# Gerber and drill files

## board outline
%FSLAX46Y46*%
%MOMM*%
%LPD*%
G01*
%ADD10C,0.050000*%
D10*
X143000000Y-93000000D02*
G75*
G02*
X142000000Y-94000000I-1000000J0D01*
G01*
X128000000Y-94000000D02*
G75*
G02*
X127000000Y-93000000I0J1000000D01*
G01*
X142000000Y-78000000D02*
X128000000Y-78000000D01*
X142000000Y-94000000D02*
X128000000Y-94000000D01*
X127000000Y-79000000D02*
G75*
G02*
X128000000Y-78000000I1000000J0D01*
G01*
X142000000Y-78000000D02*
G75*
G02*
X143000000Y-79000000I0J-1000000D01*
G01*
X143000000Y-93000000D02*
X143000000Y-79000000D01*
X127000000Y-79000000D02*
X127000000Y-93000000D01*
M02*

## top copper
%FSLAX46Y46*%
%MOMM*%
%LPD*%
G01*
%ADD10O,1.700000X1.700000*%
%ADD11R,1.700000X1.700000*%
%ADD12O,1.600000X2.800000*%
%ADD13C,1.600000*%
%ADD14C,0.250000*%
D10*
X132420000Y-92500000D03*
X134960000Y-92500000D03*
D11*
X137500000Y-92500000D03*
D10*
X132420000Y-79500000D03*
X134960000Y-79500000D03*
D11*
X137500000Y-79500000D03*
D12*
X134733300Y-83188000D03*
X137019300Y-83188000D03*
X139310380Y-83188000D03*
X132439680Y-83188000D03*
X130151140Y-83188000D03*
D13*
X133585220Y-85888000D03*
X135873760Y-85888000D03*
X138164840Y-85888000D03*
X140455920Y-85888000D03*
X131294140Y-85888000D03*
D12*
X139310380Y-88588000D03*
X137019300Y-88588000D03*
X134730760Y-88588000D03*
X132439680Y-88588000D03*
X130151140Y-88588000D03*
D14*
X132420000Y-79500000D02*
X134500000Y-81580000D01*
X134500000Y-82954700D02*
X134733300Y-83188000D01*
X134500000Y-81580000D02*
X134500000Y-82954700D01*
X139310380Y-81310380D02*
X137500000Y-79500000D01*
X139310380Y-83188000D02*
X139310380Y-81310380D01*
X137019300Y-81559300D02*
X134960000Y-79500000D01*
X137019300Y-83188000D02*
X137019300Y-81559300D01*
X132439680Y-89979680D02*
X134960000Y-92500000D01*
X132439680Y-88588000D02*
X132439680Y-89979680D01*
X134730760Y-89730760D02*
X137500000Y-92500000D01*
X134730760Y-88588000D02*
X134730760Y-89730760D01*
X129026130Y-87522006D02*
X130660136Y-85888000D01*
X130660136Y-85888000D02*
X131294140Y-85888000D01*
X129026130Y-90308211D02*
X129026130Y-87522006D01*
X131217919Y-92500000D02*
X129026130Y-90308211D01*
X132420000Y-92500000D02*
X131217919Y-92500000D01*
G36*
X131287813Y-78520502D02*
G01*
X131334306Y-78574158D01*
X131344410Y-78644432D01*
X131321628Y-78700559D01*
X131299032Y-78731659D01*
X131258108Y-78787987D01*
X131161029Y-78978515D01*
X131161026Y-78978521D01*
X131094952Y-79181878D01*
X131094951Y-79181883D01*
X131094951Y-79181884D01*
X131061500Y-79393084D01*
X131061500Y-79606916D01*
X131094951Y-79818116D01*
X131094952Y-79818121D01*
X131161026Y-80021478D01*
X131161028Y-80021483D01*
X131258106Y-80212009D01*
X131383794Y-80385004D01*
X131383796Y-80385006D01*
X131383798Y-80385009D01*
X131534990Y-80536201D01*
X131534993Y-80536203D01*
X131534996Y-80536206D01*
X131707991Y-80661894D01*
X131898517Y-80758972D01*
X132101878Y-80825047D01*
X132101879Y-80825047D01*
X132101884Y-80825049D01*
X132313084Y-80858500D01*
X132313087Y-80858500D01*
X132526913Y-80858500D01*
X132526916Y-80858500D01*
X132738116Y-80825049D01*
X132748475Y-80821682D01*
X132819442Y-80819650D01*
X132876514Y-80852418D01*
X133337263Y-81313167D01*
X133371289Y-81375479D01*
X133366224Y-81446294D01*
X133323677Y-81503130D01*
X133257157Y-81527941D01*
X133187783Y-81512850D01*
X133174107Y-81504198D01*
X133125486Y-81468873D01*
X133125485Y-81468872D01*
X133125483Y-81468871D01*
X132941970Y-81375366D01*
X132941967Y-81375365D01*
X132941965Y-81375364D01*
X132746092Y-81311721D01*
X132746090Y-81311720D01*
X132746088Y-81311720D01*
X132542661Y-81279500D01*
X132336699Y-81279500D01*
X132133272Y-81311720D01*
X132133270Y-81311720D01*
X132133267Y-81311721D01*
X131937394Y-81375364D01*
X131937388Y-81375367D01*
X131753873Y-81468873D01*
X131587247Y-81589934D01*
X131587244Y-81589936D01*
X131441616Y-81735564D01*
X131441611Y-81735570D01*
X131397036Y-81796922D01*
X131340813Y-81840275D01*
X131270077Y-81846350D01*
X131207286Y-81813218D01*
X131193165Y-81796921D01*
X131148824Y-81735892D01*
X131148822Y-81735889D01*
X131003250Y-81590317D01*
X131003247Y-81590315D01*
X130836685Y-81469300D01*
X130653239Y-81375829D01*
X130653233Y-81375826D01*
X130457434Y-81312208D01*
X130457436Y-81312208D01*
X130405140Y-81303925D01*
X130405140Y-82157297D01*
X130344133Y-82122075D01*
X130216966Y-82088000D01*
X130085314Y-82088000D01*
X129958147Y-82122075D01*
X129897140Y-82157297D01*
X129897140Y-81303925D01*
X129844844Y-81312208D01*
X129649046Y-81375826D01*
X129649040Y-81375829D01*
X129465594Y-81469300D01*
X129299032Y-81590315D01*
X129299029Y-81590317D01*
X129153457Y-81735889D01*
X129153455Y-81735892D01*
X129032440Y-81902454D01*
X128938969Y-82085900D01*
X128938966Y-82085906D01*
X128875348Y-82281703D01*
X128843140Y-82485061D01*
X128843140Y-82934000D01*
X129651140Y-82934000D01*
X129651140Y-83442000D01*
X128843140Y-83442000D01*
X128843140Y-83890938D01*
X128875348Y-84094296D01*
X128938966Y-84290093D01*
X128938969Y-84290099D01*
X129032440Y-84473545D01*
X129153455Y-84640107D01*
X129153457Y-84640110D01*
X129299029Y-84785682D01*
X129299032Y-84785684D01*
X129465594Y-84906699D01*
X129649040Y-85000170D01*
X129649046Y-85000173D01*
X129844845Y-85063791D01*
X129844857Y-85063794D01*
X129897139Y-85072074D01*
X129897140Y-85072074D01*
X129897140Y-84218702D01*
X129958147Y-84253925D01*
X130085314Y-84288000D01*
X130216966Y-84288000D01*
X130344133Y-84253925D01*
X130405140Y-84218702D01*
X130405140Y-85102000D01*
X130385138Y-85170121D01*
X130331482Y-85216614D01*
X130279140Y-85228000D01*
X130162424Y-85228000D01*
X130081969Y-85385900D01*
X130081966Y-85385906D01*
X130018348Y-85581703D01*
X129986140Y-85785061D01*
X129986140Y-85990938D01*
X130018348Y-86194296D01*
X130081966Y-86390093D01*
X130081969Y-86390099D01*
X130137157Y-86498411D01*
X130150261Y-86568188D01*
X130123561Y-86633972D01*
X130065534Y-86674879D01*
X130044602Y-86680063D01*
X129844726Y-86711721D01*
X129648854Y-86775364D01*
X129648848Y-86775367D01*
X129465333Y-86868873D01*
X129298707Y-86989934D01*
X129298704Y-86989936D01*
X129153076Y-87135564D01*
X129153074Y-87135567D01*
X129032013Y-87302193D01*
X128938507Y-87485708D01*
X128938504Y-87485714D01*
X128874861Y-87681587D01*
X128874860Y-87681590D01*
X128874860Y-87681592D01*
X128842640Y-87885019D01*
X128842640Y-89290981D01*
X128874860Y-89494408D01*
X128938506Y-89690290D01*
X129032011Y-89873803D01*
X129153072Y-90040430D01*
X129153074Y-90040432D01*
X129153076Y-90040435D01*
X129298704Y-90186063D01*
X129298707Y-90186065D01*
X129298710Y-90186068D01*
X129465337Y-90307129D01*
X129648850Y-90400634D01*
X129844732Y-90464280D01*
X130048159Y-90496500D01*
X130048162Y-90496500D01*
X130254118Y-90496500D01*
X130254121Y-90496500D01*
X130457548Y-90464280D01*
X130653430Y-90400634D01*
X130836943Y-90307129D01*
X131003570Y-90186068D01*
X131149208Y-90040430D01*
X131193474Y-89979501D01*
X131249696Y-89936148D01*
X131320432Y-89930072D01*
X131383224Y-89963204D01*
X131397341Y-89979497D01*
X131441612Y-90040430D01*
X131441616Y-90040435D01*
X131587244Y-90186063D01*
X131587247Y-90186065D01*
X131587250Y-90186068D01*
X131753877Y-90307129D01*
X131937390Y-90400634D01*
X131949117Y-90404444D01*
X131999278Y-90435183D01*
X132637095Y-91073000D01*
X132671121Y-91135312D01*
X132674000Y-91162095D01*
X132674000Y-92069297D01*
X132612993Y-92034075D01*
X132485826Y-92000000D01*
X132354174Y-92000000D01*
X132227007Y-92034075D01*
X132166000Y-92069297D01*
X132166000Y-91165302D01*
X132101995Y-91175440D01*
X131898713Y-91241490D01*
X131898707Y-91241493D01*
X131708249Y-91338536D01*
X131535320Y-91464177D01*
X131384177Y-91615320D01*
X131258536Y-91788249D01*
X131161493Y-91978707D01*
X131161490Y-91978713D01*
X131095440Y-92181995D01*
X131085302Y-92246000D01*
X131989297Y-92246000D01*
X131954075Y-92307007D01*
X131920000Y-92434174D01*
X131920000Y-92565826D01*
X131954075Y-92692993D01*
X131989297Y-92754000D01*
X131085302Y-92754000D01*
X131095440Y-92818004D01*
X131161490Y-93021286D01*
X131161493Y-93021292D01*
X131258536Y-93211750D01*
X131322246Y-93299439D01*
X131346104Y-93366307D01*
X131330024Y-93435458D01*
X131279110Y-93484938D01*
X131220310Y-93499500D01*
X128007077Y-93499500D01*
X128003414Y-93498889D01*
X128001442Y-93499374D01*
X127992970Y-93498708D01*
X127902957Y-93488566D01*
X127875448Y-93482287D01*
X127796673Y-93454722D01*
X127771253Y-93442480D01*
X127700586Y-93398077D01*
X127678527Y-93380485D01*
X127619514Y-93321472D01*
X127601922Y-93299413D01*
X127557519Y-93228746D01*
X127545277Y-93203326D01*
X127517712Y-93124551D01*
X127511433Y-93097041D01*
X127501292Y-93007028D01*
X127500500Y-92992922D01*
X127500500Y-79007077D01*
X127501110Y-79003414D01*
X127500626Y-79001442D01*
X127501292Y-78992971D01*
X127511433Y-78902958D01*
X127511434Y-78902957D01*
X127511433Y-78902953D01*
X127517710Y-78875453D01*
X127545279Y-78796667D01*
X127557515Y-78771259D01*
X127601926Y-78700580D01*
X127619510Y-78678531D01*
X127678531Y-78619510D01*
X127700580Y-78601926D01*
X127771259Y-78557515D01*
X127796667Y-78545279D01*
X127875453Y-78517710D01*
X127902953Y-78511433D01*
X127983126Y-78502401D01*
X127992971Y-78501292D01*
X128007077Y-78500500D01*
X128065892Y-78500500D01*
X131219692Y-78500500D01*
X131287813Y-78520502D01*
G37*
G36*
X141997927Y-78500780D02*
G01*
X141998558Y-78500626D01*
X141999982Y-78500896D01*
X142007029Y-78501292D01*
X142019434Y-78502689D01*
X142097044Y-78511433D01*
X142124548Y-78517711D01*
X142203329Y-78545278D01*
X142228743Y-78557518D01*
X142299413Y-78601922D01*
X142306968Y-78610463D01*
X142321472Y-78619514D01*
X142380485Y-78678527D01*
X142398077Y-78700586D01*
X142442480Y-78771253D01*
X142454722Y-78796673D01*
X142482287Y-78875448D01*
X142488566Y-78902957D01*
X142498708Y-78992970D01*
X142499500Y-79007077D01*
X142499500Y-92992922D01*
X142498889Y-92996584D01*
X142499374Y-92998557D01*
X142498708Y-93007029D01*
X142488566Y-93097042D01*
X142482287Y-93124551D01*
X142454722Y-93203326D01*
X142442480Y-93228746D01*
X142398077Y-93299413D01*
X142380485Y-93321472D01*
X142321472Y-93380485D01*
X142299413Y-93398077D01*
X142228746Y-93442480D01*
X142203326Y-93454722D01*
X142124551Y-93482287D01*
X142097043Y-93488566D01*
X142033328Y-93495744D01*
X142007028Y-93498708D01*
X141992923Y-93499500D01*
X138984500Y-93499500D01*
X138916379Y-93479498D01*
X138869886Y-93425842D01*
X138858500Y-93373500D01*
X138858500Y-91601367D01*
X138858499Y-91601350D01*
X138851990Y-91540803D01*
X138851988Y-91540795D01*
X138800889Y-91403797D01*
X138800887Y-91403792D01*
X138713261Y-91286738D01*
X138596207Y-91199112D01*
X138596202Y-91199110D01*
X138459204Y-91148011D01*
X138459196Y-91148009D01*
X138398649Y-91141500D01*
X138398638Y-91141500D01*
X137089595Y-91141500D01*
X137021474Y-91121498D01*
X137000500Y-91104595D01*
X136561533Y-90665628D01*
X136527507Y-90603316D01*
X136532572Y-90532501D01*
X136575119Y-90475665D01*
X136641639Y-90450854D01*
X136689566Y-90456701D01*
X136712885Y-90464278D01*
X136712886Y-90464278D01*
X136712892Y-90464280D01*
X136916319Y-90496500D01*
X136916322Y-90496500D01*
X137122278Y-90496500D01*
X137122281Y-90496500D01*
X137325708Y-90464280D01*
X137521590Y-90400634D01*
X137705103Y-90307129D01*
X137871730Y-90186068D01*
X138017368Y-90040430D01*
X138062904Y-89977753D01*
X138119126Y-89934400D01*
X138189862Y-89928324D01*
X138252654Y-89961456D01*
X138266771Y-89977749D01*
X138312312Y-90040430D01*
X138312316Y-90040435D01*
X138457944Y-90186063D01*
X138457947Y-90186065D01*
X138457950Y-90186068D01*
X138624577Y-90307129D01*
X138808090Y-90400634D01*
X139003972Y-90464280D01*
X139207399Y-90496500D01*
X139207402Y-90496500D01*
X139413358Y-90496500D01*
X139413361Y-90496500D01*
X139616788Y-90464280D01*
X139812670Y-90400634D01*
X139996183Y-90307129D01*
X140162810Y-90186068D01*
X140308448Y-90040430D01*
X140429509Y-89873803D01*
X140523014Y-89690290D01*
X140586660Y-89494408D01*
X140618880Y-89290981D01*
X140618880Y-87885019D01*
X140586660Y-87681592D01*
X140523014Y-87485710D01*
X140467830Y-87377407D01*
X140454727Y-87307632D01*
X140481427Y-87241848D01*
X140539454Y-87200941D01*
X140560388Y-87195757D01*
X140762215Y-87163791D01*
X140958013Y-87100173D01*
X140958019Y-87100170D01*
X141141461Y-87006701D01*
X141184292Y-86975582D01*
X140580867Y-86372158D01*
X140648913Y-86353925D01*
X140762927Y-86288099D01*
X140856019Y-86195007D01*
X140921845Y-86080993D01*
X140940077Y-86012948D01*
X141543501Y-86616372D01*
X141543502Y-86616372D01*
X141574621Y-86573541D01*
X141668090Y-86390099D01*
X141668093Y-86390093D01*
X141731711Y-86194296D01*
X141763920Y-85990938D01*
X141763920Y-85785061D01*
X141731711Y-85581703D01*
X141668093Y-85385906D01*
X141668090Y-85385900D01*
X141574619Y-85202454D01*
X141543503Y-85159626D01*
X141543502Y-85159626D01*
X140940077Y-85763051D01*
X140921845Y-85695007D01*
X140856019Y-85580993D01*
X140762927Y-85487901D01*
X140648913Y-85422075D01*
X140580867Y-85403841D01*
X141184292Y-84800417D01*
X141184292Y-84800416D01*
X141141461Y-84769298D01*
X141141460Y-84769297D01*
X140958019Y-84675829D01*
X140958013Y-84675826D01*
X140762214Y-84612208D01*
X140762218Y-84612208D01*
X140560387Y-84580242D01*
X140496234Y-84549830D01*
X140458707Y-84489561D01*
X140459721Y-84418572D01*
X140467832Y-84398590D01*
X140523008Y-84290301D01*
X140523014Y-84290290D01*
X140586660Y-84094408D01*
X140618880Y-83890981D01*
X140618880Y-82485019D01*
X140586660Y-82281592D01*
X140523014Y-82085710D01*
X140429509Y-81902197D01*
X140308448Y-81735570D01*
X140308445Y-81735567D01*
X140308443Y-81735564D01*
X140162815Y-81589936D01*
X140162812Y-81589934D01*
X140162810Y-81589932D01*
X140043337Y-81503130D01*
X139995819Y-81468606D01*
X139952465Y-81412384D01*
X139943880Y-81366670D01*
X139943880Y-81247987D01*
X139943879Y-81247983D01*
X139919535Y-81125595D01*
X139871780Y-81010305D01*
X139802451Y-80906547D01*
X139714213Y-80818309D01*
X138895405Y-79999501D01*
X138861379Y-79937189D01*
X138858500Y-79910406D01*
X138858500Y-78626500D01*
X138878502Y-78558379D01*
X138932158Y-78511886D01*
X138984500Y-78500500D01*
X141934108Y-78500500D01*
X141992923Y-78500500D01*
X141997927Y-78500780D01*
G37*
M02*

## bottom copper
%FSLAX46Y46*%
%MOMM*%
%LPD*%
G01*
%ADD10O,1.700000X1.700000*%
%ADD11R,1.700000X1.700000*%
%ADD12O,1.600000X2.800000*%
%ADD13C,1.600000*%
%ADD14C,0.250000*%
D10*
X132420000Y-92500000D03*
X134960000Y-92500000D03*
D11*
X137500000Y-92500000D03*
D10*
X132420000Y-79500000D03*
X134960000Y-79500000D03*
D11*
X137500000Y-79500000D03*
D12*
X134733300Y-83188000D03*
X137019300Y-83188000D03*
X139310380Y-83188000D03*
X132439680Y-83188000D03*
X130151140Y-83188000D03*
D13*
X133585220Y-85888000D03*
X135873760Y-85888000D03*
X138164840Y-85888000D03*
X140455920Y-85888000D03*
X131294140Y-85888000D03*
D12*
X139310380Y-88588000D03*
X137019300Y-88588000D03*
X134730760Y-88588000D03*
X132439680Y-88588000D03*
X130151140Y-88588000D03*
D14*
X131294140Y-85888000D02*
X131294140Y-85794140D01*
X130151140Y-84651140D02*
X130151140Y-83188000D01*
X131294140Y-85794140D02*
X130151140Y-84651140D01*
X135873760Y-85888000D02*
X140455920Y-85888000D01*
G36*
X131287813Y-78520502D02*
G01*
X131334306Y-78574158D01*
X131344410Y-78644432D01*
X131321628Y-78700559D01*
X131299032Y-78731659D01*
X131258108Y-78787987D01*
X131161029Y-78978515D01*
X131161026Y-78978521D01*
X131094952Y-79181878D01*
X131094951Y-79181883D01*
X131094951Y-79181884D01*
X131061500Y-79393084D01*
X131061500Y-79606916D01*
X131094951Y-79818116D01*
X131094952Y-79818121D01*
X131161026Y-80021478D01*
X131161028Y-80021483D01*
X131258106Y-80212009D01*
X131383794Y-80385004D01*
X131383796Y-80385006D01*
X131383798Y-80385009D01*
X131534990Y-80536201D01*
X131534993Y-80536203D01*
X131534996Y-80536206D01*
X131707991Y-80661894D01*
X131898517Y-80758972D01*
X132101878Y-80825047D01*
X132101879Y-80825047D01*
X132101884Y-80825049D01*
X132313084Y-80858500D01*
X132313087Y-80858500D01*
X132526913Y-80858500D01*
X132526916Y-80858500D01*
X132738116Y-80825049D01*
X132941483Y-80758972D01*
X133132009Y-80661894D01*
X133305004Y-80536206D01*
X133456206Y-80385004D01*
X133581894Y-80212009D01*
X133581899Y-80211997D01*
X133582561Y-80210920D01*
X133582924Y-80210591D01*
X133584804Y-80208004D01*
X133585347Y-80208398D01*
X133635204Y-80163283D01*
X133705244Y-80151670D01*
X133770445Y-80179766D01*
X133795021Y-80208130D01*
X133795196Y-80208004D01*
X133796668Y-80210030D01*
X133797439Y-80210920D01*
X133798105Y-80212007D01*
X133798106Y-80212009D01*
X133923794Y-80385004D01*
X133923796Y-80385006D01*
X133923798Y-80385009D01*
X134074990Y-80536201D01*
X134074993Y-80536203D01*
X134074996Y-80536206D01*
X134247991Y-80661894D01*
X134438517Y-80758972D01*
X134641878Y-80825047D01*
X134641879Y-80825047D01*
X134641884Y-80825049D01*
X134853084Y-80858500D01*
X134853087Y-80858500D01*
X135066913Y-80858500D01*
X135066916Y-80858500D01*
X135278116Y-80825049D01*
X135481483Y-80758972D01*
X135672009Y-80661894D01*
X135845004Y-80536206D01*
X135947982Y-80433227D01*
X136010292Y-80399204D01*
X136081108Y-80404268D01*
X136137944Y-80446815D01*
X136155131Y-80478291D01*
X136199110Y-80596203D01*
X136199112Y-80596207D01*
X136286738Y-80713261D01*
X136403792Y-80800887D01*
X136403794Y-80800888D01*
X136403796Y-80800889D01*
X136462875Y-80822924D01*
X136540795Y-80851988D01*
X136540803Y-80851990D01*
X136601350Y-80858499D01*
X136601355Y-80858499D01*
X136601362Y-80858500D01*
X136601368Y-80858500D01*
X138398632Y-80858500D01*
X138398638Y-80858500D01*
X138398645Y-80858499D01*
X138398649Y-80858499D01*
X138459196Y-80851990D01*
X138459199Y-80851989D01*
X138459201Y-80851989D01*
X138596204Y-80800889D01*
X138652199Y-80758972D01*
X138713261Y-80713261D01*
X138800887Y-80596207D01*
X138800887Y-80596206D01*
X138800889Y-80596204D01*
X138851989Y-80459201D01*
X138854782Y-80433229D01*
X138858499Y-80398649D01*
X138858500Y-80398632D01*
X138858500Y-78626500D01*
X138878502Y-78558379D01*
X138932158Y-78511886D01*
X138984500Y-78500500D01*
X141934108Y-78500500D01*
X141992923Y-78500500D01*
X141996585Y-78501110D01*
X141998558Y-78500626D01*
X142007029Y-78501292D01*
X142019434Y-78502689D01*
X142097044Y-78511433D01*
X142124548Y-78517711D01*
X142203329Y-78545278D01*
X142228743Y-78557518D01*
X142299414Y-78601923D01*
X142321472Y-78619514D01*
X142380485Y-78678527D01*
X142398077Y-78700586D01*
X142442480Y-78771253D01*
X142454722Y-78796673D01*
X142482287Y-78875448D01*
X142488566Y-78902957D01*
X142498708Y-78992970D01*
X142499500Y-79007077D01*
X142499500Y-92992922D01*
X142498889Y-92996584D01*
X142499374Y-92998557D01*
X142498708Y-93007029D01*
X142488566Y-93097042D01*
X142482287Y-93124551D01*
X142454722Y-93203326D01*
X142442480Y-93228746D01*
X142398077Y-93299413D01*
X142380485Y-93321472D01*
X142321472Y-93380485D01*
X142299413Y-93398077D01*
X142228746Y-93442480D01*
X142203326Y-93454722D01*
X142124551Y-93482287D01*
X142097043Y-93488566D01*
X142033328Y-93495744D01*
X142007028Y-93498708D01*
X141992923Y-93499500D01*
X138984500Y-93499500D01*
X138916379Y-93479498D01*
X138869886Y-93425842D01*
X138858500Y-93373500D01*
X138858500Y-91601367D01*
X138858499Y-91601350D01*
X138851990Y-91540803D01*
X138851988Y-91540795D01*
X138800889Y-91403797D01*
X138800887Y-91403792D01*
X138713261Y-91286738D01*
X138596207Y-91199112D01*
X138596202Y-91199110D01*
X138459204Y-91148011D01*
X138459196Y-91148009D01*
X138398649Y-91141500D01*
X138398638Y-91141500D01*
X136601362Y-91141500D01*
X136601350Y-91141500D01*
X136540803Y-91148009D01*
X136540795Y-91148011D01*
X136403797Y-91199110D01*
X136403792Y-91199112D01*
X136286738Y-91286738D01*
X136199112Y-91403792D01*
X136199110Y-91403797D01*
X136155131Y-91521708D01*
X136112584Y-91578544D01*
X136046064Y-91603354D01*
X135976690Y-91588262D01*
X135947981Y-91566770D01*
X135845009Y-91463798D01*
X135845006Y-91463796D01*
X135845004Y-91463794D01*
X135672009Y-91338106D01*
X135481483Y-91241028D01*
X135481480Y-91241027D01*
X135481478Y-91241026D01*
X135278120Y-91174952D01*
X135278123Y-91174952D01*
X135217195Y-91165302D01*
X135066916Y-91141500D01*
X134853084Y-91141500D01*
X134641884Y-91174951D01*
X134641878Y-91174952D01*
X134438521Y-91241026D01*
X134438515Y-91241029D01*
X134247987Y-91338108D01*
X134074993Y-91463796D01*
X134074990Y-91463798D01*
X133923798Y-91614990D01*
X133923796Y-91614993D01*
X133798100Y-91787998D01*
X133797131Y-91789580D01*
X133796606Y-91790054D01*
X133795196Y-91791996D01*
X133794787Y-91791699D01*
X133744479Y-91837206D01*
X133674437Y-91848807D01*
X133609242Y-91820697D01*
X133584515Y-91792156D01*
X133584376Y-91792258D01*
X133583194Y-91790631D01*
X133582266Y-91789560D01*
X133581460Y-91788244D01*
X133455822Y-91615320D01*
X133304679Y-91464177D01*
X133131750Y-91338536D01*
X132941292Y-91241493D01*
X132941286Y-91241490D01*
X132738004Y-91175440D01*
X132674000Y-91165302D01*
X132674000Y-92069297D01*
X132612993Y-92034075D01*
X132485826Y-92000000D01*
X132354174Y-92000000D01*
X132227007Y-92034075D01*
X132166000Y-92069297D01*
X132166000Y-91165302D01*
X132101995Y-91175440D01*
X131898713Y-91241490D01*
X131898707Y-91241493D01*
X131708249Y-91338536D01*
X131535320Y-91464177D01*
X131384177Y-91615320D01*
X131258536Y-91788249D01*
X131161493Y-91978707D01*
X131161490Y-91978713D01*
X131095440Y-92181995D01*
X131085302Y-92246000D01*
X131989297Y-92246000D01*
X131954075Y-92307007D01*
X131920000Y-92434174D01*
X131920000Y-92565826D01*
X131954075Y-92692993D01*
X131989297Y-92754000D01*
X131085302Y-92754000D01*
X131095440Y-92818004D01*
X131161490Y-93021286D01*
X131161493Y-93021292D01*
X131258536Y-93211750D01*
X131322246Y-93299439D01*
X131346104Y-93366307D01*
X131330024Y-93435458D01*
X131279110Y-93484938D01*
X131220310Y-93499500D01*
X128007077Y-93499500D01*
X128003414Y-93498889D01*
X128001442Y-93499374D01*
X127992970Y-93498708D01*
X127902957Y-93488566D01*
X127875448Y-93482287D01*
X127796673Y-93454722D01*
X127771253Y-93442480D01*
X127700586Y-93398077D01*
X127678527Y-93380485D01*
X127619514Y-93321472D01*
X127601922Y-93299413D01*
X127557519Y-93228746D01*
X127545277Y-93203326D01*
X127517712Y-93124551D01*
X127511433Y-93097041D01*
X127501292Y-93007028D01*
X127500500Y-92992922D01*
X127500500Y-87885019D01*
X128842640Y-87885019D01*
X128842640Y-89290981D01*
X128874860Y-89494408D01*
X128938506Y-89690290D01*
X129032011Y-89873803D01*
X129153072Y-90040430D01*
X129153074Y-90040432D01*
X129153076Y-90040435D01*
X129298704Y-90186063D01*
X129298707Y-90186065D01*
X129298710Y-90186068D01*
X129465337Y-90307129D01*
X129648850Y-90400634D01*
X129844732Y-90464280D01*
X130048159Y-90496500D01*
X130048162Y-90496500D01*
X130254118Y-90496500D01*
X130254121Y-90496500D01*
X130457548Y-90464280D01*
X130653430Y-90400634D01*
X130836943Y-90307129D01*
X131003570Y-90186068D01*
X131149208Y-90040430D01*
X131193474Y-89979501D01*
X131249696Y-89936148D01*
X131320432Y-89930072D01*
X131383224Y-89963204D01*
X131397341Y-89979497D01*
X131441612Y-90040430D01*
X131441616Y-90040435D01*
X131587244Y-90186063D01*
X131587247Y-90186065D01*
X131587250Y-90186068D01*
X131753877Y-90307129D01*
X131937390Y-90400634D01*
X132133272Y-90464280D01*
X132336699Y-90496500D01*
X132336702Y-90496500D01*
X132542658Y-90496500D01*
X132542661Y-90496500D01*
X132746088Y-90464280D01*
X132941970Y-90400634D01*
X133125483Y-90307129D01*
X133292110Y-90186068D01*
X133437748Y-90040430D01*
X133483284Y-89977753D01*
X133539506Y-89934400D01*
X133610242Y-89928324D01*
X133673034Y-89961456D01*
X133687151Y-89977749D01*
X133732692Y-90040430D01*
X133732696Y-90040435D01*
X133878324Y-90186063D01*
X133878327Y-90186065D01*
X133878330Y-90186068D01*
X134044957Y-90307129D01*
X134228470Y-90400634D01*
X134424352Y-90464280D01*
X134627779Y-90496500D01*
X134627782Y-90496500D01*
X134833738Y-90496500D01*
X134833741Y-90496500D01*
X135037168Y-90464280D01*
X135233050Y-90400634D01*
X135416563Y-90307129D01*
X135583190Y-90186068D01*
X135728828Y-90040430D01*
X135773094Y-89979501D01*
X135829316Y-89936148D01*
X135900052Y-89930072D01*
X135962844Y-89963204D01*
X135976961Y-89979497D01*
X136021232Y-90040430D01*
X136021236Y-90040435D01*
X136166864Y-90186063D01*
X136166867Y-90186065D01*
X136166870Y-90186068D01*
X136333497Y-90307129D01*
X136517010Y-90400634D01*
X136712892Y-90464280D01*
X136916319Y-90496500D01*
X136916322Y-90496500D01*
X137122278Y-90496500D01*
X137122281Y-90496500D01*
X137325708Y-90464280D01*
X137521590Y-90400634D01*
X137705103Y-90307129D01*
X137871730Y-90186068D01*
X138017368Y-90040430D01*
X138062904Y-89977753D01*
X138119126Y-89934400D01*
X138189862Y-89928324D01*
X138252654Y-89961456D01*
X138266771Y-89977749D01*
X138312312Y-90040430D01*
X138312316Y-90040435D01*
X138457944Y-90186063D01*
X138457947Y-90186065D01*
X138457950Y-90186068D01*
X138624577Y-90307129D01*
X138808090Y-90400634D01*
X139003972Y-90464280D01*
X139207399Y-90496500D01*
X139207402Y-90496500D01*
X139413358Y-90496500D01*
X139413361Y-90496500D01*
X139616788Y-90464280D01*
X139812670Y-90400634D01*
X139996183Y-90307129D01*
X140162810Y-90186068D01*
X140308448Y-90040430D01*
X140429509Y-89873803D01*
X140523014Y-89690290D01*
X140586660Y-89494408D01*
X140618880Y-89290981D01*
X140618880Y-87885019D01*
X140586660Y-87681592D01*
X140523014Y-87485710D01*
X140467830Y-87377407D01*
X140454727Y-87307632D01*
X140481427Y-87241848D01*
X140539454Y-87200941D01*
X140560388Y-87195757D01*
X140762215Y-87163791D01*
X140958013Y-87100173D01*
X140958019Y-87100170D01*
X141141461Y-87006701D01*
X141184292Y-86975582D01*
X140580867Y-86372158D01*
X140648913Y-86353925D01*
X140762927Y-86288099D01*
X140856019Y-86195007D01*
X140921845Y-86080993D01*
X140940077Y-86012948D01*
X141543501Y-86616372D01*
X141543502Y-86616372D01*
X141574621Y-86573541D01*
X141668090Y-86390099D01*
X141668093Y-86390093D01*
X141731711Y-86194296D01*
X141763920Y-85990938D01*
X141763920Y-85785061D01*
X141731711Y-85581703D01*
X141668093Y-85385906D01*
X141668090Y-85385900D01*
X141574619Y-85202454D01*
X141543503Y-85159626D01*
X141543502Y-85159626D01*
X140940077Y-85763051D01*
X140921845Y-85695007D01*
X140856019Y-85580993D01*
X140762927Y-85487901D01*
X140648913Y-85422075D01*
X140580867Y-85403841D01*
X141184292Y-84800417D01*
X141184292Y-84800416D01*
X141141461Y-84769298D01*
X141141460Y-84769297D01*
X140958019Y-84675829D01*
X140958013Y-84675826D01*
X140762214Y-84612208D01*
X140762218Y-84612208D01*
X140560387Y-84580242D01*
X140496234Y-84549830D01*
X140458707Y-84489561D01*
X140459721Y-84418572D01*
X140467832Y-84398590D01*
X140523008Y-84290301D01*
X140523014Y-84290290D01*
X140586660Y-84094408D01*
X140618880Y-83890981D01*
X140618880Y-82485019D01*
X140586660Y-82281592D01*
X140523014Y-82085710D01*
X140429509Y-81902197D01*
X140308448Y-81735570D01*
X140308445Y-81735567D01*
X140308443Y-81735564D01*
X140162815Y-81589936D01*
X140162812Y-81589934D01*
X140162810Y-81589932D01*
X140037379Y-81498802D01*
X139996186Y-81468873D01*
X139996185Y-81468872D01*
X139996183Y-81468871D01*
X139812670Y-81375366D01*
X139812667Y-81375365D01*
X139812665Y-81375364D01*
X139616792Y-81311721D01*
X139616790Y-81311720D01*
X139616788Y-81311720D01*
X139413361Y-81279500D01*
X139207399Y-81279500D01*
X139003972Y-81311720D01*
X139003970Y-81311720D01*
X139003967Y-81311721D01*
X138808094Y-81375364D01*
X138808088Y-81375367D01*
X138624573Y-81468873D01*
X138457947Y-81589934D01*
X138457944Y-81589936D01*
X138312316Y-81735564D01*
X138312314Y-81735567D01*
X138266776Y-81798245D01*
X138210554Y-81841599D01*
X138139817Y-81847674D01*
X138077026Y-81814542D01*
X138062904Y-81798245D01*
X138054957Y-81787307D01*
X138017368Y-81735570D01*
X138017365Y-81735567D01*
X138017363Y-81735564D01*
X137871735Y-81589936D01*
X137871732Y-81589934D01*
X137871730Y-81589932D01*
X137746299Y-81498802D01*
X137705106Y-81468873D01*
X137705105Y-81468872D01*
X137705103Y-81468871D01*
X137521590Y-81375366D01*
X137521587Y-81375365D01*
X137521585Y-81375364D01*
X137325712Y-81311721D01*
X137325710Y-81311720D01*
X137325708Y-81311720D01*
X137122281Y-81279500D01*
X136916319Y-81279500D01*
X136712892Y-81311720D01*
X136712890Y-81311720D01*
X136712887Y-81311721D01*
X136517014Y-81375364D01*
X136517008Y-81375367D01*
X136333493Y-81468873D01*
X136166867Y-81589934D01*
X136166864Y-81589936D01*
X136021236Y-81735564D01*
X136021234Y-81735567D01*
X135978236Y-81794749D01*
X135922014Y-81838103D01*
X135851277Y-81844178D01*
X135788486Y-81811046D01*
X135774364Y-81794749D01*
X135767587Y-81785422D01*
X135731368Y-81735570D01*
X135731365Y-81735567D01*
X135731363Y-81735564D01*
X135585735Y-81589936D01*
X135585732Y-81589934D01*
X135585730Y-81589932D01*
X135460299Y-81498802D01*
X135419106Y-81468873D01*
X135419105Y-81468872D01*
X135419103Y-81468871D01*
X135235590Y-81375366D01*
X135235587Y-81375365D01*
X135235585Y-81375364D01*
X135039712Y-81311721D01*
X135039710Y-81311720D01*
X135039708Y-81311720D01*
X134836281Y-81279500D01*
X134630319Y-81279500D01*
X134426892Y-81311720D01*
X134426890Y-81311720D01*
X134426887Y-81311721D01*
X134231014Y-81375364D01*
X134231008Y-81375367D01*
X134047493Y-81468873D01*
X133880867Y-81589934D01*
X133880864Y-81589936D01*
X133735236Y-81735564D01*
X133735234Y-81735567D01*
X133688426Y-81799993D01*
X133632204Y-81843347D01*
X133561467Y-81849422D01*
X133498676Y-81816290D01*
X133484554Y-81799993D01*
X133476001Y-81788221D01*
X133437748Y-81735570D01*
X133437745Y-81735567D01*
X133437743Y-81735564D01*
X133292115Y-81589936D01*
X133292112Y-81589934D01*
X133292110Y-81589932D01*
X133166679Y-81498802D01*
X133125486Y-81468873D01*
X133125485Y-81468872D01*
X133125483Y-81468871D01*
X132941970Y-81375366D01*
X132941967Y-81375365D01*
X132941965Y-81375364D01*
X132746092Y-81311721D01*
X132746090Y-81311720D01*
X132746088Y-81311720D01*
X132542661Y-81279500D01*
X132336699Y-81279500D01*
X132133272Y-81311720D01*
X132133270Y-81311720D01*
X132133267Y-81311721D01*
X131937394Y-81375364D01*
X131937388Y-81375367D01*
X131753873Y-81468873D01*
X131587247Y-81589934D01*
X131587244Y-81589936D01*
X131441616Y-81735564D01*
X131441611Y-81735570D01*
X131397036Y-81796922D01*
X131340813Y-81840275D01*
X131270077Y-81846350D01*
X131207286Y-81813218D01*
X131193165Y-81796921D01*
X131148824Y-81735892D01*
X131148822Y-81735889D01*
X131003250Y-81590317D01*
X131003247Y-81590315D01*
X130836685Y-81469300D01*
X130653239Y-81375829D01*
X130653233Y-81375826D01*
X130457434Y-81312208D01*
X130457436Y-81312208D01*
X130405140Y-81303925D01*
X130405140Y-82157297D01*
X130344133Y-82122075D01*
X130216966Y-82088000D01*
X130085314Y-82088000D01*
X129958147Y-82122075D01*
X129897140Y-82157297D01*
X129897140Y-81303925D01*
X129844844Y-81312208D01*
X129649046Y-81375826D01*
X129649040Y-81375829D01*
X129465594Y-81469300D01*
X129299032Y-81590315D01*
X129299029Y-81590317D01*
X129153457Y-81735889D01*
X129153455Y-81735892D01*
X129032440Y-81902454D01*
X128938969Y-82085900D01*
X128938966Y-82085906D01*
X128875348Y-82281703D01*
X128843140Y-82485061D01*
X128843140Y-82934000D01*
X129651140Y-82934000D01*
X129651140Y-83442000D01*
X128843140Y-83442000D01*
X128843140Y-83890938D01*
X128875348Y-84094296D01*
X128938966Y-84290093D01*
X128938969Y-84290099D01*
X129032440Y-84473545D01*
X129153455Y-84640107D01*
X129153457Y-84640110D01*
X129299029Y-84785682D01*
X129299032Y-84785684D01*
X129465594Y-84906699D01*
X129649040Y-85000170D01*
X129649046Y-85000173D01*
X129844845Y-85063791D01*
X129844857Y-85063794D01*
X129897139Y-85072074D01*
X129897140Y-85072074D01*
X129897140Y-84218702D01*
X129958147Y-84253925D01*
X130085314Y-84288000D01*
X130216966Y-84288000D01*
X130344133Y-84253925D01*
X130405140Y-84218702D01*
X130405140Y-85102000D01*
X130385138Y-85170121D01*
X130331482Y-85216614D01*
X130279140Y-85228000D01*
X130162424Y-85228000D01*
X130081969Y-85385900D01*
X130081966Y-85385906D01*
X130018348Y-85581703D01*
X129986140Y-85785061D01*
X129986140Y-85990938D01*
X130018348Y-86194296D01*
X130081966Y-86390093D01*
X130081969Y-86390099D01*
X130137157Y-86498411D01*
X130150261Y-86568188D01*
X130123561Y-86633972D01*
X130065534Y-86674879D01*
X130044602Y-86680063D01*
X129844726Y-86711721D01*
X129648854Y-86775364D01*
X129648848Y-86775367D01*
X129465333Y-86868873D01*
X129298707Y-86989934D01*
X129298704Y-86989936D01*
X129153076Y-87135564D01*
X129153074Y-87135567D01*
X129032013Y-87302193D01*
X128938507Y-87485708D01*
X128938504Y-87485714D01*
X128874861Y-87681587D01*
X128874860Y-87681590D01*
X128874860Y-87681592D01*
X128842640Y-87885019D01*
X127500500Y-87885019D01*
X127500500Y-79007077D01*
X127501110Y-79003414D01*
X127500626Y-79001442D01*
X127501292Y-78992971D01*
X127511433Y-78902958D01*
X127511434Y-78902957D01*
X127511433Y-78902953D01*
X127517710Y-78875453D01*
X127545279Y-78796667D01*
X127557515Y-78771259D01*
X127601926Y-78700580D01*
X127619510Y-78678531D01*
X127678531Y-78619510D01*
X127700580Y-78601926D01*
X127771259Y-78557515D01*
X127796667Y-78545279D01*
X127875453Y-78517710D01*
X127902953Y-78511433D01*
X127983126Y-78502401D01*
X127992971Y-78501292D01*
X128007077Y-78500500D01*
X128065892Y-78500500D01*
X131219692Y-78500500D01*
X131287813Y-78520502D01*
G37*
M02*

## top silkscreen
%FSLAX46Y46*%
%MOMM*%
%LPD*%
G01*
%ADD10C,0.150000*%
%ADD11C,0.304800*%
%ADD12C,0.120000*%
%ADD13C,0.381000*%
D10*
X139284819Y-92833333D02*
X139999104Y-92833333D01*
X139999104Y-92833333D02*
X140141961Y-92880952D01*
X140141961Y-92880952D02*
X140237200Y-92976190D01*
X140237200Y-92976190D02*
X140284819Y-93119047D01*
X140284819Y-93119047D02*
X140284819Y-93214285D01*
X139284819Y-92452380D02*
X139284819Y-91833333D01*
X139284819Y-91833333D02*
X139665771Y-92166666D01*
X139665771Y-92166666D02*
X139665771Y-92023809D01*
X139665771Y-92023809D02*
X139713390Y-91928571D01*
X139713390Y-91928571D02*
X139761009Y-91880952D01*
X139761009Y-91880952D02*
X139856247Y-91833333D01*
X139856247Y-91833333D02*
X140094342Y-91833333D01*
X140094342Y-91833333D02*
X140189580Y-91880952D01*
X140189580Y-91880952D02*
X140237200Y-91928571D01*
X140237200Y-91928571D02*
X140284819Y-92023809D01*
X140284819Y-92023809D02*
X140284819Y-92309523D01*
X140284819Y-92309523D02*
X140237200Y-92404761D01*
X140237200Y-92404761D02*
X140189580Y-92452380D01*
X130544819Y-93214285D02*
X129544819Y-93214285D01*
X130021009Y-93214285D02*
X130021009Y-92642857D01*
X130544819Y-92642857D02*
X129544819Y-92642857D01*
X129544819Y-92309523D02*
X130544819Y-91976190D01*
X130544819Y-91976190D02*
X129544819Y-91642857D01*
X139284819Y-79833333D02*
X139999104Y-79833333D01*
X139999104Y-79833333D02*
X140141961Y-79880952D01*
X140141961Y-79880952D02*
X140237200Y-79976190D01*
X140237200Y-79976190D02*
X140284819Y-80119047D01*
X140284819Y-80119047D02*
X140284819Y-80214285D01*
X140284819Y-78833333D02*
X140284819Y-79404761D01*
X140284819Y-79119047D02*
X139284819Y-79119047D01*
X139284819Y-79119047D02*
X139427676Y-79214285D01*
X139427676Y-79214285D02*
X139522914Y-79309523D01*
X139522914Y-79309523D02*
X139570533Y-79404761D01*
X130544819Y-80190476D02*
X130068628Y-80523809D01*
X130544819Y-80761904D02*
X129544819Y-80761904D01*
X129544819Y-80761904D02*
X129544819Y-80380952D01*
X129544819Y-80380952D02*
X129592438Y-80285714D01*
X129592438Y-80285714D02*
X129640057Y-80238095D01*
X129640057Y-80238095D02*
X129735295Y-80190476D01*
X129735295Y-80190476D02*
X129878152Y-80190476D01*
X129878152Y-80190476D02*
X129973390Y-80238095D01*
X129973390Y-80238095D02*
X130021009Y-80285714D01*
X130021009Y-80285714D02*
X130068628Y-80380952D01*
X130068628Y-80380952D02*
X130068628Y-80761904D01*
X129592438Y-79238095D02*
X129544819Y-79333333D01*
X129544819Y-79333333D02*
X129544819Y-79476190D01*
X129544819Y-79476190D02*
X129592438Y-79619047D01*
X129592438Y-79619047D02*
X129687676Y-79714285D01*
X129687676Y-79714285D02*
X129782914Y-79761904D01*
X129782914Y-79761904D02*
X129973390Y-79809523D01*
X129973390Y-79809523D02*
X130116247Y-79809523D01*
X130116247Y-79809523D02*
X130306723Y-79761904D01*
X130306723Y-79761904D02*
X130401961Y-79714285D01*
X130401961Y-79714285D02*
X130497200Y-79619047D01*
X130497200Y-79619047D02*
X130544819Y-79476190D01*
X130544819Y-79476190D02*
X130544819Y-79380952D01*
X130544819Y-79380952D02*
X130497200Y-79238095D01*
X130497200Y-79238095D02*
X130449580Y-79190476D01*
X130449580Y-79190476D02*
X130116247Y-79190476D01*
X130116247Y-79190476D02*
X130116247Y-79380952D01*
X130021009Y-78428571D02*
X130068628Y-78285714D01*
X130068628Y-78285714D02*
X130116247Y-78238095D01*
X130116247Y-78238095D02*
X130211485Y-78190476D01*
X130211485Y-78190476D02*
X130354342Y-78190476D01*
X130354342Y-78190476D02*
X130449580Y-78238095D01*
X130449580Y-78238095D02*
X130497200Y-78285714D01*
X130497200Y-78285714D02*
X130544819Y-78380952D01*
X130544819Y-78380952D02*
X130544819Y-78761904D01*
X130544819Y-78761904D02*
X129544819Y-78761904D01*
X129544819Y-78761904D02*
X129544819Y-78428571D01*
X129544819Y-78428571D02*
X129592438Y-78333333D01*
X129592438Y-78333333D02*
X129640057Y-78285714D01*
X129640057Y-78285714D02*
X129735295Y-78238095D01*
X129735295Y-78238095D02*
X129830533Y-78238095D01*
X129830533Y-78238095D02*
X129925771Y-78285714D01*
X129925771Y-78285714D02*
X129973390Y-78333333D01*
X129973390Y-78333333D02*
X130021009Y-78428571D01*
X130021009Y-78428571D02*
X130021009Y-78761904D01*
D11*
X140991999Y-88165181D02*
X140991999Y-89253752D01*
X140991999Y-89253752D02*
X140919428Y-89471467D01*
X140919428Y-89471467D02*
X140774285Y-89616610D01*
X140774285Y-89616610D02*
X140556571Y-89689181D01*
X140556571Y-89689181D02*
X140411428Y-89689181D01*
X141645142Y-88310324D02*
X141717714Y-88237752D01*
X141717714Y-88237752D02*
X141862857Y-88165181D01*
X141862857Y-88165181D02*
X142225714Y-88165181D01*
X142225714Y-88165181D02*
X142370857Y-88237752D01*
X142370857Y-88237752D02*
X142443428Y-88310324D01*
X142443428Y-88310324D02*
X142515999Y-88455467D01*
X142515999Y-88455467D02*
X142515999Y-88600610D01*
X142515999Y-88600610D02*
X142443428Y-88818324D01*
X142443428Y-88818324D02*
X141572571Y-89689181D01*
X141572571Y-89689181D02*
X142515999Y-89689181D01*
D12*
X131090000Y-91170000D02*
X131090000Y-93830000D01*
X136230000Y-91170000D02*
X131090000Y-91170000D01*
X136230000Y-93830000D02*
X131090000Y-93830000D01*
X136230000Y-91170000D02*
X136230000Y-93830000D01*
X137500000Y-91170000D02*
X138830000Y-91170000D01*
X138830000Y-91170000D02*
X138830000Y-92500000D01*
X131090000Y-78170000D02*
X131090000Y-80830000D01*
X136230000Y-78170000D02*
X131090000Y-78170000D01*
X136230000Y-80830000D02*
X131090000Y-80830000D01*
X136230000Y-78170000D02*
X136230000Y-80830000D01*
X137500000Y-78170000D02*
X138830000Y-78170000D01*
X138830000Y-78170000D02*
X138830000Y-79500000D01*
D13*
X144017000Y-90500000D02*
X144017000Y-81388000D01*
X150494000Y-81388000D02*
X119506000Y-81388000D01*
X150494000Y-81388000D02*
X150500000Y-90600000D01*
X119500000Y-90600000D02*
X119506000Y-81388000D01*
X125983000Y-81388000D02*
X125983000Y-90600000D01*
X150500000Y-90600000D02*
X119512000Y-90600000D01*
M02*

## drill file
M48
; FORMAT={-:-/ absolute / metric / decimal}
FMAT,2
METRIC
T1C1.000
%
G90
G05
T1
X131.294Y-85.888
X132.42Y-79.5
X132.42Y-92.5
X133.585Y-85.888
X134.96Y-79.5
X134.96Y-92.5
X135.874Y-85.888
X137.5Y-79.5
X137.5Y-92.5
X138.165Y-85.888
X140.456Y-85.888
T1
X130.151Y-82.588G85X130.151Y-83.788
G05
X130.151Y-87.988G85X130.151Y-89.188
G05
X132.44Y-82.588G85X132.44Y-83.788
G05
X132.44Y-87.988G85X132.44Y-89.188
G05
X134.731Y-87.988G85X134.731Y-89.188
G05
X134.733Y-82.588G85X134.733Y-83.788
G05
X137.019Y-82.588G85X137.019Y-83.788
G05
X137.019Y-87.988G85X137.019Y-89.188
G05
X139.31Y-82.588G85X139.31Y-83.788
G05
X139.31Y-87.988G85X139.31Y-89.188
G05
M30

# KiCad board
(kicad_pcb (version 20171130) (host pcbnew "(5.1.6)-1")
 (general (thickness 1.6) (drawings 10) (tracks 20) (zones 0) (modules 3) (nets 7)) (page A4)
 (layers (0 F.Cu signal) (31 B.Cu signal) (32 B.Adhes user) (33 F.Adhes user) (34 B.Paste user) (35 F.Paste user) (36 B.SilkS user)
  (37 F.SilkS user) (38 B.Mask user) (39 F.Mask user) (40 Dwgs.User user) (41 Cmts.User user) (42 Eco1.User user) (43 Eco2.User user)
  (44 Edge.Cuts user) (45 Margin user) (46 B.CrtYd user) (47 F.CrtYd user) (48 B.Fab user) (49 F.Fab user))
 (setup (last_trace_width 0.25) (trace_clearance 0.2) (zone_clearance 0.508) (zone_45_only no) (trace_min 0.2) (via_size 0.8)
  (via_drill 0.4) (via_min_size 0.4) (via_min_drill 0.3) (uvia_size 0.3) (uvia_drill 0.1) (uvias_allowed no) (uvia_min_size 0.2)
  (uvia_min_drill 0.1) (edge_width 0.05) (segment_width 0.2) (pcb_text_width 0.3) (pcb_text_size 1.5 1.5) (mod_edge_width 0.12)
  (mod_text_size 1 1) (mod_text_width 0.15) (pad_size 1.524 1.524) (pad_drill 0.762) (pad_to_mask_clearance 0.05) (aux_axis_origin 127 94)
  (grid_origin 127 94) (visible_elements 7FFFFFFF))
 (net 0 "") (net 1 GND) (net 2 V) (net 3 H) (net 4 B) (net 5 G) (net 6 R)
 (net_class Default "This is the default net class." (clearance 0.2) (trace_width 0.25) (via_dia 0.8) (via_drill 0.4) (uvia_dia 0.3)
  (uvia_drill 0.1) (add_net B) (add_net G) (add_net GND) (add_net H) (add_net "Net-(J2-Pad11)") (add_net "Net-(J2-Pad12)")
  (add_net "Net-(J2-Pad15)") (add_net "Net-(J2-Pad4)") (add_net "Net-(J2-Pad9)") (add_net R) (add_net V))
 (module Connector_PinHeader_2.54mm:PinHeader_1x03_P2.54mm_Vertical (layer F.Cu) (at 137.5 92.5 270)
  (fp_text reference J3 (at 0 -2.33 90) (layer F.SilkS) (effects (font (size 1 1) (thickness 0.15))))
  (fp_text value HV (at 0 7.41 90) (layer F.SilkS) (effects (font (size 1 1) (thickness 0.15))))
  (fp_line (start -1.33 6.41) (end 1.33 6.41) (layer F.SilkS) (width 0.12))
  (fp_line (start -1.33 1.27) (end -1.33 6.41) (layer F.SilkS) (width 0.12))
  (fp_line (start 1.33 1.27) (end 1.33 6.41) (layer F.SilkS) (width 0.12))
  (fp_line (start -1.33 1.27) (end 1.33 1.27) (layer F.SilkS) (width 0.12))
  (fp_line (start -1.33 0) (end -1.33 -1.33) (layer F.SilkS) (width 0.12))
  (fp_line (start -1.33 -1.33) (end 0 -1.33) (layer F.SilkS) (width 0.12))
  (pad 3 thru_hole oval (at 0 5.08 270) (size 1.7 1.7) (drill 1) (layers *.Cu *.Mask) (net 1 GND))
  (pad 2 thru_hole oval (at 0 2.54 270) (size 1.7 1.7) (drill 1) (layers *.Cu *.Mask) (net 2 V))
  (pad 1 thru_hole rect (at 0 0 270) (size 1.7 1.7) (drill 1) (layers *.Cu *.Mask) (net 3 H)))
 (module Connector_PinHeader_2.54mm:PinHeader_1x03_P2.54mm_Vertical (layer F.Cu) (at 137.5 79.5 270)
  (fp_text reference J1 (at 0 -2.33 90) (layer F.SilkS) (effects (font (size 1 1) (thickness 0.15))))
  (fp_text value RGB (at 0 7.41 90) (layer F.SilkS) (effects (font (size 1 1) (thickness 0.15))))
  (fp_line (start -1.33 6.41) (end 1.33 6.41) (layer F.SilkS) (width 0.12))
  (fp_line (start -1.33 1.27) (end -1.33 6.41) (layer F.SilkS) (width 0.12))
  (fp_line (start 1.33 1.27) (end 1.33 6.41) (layer F.SilkS) (width 0.12))
  (fp_line (start -1.33 1.27) (end 1.33 1.27) (layer F.SilkS) (width 0.12))
  (fp_line (start -1.33 0) (end -1.33 -1.33) (layer F.SilkS) (width 0.12))
  (fp_line (start -1.33 -1.33) (end 0 -1.33) (layer F.SilkS) (width 0.12))
  (pad 3 thru_hole oval (at 0 5.08 270) (size 1.7 1.7) (drill 1) (layers *.Cu *.Mask) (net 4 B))
  (pad 2 thru_hole oval (at 0 2.54 270) (size 1.7 1.7) (drill 1) (layers *.Cu *.Mask) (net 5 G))
  (pad 1 thru_hole rect (at 0 0 270) (size 1.7 1.7) (drill 1) (layers *.Cu *.Mask) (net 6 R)))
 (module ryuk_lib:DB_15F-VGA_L (layer F.Cu) (at 135 96.5)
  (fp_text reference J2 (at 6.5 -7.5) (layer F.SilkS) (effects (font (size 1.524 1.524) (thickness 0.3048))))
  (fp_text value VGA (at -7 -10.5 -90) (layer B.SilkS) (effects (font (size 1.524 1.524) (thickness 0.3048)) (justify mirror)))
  (fp_line (start 9.017 -6) (end 9.017 -15.112) (layer F.SilkS) (width 0.381))
  (fp_line (start 15.494 -15.112) (end -15.494 -15.112) (layer F.SilkS) (width 0.381))
  (fp_line (start 15.494 -15.112) (end 15.5 -5.9) (layer F.SilkS) (width 0.381))
  (fp_line (start -15.5 -5.9) (end -15.494 -15.112) (layer F.SilkS) (width 0.381))
  (fp_line (start -9.017 -15.112) (end -9.017 -5.9) (layer F.SilkS) (width 0.381))
  (fp_line (start 15.5 -5.9) (end -15.488 -5.9) (layer F.SilkS) (width 0.381))
  (pad 3 thru_hole oval (at -0.2667 -13.312) (size 1.6 2.8) (drill oval 1 2.2) (layers *.Cu *.Mask) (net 4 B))
  (pad 2 thru_hole oval (at 2.0193 -13.312) (size 1.6 2.8) (drill oval 1 2.2) (layers *.Cu *.Mask) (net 5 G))
  (pad 1 thru_hole oval (at 4.31038 -13.312) (size 1.6 2.8) (drill oval 1 2.2) (layers *.Cu *.Mask) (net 6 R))
  (pad 4 thru_hole oval (at -2.56032 -13.312) (size 1.6 2.8) (drill oval 1 2.2) (layers *.Cu *.Mask))
  (pad 5 thru_hole oval (at -4.84886 -13.312) (size 1.6 2.8) (drill oval 1 2.2) (layers *.Cu *.Mask) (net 1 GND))
  (pad 9 thru_hole circle (at -1.41478 -10.612) (size 1.6 1.6) (drill 1) (layers *.Cu *.Mask))
  (pad 8 thru_hole circle (at 0.87376 -10.612) (size 1.6 1.6) (drill 1) (layers *.Cu *.Mask) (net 1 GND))
  (pad 7 thru_hole circle (at 3.16484 -10.612) (size 1.6 1.6) (drill 1) (layers *.Cu *.Mask) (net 1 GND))
  (pad 6 thru_hole circle (at 5.45592 -10.612) (size 1.6 1.6) (drill 1) (layers *.Cu *.Mask) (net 1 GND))
  (pad 10 thru_hole circle (at -3.70586 -10.612) (size 1.6 1.6) (drill 1) (layers *.Cu *.Mask) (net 1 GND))
  (pad 11 thru_hole oval (at 4.31038 -7.912) (size 1.6 2.8) (drill oval 1 2.2) (layers *.Cu *.Mask))
  (pad 12 thru_hole oval (at 2.0193 -7.912) (size 1.6 2.8) (drill oval 1 2.2) (layers *.Cu *.Mask))
  (pad 13 thru_hole oval (at -0.26924 -7.912) (size 1.6 2.8) (drill oval 1 2.2) (layers *.Cu *.Mask) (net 3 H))
  (pad 14 thru_hole oval (at -2.56032 -7.912) (size 1.6 2.8) (drill oval 1 2.2) (layers *.Cu *.Mask) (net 2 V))
  (pad 15 thru_hole oval (at -4.84886 -7.912) (size 1.6 2.8) (drill oval 1 2.2) (layers *.Cu *.Mask)))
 (gr_arc (start 142 93) (end 142 94) (angle -90) (layer Edge.Cuts) (width 0.05))
 (gr_arc (start 128 93) (end 127 93) (angle -90) (layer Edge.Cuts) (width 0.05))
 (gr_line (start 142 78) (end 128 78) (layer Edge.Cuts) (width 0.05))
 (gr_line (start 142 94) (end 128 94) (layer Edge.Cuts) (width 0.05))
 (gr_arc (start 128 79) (end 128 78) (angle -90) (layer Edge.Cuts) (width 0.05))
 (gr_arc (start 142 79) (end 143 79) (angle -90) (layer Edge.Cuts) (width 0.05))
 (gr_line (start 143 93) (end 143 79) (layer Edge.Cuts) (width 0.05))
 (gr_line (start 127 79) (end 127 93) (layer Edge.Cuts) (width 0.05))
 (segment (start 132.42 79.5) (end 134.5 81.58) (width 0.25) (layer F.Cu) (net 4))
 (segment (start 134.5 82.9547) (end 134.7333 83.188) (width 0.25) (layer F.Cu) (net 4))
 (segment (start 134.5 81.58) (end 134.5 82.9547) (width 0.25) (layer F.Cu) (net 4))
 (segment (start 139.31038 81.31038) (end 137.5 79.5) (width 0.25) (layer F.Cu) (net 6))
 (segment (start 139.31038 83.188) (end 139.31038 81.31038) (width 0.25) (layer F.Cu) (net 6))
 (segment (start 137.0193 81.5593) (end 134.96 79.5) (width 0.25) (layer F.Cu) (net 5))
 (segment (start 137.0193 83.188) (end 137.0193 81.5593) (width 0.25) (layer F.Cu) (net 5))
 (segment (start 132.43968 89.97968) (end 134.96 92.5) (width 0.25) (layer F.Cu) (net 2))
 (segment (start 132.43968 88.588) (end 132.43968 89.97968) (width 0.25) (layer F.Cu) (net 2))
 (segment (start 134.73076 89.73076) (end 137.5 92.5) (width 0.25) (layer F.Cu) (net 3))
 (segment (start 134.73076 88.588) (end 134.73076 89.73076) (width 0.25) (layer F.Cu) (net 3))
 (segment (start 129.02613 87.522006) (end 130.660136 85.888) (width 0.25) (layer F.Cu) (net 1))
 (segment (start 130.660136 85.888) (end 131.29414 85.888) (width 0.25) (layer F.Cu) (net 1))
 (segment (start 129.02613 90.308211) (end 129.02613 87.522006) (width 0.25) (layer F.Cu) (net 1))
 (segment (start 131.217919 92.5) (end 129.02613 90.308211) (width 0.25) (layer F.Cu) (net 1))
 (segment (start 132.42 92.5) (end 131.217919 92.5) (width 0.25) (layer F.Cu) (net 1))
 (segment (start 131.29414 85.888) (end 131.29414 85.79414) (width 0.25) (layer B.Cu) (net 1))
 (segment (start 130.15114 84.65114) (end 130.15114 83.188) (width 0.25) (layer B.Cu) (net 1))
 (segment (start 131.29414 85.79414) (end 130.15114 84.65114) (width 0.25) (layer B.Cu) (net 1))
 (segment (start 135.87376 85.888) (end 140.45592 85.888) (width 0.25) (layer B.Cu) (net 1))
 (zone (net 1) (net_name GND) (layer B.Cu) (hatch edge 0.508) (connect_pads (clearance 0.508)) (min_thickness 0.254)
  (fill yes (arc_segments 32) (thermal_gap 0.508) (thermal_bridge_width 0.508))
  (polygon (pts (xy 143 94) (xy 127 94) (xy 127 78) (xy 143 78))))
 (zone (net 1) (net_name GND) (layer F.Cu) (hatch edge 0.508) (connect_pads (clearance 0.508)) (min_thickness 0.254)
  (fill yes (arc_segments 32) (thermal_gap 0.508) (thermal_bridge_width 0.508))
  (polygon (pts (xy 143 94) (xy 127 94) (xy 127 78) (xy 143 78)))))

